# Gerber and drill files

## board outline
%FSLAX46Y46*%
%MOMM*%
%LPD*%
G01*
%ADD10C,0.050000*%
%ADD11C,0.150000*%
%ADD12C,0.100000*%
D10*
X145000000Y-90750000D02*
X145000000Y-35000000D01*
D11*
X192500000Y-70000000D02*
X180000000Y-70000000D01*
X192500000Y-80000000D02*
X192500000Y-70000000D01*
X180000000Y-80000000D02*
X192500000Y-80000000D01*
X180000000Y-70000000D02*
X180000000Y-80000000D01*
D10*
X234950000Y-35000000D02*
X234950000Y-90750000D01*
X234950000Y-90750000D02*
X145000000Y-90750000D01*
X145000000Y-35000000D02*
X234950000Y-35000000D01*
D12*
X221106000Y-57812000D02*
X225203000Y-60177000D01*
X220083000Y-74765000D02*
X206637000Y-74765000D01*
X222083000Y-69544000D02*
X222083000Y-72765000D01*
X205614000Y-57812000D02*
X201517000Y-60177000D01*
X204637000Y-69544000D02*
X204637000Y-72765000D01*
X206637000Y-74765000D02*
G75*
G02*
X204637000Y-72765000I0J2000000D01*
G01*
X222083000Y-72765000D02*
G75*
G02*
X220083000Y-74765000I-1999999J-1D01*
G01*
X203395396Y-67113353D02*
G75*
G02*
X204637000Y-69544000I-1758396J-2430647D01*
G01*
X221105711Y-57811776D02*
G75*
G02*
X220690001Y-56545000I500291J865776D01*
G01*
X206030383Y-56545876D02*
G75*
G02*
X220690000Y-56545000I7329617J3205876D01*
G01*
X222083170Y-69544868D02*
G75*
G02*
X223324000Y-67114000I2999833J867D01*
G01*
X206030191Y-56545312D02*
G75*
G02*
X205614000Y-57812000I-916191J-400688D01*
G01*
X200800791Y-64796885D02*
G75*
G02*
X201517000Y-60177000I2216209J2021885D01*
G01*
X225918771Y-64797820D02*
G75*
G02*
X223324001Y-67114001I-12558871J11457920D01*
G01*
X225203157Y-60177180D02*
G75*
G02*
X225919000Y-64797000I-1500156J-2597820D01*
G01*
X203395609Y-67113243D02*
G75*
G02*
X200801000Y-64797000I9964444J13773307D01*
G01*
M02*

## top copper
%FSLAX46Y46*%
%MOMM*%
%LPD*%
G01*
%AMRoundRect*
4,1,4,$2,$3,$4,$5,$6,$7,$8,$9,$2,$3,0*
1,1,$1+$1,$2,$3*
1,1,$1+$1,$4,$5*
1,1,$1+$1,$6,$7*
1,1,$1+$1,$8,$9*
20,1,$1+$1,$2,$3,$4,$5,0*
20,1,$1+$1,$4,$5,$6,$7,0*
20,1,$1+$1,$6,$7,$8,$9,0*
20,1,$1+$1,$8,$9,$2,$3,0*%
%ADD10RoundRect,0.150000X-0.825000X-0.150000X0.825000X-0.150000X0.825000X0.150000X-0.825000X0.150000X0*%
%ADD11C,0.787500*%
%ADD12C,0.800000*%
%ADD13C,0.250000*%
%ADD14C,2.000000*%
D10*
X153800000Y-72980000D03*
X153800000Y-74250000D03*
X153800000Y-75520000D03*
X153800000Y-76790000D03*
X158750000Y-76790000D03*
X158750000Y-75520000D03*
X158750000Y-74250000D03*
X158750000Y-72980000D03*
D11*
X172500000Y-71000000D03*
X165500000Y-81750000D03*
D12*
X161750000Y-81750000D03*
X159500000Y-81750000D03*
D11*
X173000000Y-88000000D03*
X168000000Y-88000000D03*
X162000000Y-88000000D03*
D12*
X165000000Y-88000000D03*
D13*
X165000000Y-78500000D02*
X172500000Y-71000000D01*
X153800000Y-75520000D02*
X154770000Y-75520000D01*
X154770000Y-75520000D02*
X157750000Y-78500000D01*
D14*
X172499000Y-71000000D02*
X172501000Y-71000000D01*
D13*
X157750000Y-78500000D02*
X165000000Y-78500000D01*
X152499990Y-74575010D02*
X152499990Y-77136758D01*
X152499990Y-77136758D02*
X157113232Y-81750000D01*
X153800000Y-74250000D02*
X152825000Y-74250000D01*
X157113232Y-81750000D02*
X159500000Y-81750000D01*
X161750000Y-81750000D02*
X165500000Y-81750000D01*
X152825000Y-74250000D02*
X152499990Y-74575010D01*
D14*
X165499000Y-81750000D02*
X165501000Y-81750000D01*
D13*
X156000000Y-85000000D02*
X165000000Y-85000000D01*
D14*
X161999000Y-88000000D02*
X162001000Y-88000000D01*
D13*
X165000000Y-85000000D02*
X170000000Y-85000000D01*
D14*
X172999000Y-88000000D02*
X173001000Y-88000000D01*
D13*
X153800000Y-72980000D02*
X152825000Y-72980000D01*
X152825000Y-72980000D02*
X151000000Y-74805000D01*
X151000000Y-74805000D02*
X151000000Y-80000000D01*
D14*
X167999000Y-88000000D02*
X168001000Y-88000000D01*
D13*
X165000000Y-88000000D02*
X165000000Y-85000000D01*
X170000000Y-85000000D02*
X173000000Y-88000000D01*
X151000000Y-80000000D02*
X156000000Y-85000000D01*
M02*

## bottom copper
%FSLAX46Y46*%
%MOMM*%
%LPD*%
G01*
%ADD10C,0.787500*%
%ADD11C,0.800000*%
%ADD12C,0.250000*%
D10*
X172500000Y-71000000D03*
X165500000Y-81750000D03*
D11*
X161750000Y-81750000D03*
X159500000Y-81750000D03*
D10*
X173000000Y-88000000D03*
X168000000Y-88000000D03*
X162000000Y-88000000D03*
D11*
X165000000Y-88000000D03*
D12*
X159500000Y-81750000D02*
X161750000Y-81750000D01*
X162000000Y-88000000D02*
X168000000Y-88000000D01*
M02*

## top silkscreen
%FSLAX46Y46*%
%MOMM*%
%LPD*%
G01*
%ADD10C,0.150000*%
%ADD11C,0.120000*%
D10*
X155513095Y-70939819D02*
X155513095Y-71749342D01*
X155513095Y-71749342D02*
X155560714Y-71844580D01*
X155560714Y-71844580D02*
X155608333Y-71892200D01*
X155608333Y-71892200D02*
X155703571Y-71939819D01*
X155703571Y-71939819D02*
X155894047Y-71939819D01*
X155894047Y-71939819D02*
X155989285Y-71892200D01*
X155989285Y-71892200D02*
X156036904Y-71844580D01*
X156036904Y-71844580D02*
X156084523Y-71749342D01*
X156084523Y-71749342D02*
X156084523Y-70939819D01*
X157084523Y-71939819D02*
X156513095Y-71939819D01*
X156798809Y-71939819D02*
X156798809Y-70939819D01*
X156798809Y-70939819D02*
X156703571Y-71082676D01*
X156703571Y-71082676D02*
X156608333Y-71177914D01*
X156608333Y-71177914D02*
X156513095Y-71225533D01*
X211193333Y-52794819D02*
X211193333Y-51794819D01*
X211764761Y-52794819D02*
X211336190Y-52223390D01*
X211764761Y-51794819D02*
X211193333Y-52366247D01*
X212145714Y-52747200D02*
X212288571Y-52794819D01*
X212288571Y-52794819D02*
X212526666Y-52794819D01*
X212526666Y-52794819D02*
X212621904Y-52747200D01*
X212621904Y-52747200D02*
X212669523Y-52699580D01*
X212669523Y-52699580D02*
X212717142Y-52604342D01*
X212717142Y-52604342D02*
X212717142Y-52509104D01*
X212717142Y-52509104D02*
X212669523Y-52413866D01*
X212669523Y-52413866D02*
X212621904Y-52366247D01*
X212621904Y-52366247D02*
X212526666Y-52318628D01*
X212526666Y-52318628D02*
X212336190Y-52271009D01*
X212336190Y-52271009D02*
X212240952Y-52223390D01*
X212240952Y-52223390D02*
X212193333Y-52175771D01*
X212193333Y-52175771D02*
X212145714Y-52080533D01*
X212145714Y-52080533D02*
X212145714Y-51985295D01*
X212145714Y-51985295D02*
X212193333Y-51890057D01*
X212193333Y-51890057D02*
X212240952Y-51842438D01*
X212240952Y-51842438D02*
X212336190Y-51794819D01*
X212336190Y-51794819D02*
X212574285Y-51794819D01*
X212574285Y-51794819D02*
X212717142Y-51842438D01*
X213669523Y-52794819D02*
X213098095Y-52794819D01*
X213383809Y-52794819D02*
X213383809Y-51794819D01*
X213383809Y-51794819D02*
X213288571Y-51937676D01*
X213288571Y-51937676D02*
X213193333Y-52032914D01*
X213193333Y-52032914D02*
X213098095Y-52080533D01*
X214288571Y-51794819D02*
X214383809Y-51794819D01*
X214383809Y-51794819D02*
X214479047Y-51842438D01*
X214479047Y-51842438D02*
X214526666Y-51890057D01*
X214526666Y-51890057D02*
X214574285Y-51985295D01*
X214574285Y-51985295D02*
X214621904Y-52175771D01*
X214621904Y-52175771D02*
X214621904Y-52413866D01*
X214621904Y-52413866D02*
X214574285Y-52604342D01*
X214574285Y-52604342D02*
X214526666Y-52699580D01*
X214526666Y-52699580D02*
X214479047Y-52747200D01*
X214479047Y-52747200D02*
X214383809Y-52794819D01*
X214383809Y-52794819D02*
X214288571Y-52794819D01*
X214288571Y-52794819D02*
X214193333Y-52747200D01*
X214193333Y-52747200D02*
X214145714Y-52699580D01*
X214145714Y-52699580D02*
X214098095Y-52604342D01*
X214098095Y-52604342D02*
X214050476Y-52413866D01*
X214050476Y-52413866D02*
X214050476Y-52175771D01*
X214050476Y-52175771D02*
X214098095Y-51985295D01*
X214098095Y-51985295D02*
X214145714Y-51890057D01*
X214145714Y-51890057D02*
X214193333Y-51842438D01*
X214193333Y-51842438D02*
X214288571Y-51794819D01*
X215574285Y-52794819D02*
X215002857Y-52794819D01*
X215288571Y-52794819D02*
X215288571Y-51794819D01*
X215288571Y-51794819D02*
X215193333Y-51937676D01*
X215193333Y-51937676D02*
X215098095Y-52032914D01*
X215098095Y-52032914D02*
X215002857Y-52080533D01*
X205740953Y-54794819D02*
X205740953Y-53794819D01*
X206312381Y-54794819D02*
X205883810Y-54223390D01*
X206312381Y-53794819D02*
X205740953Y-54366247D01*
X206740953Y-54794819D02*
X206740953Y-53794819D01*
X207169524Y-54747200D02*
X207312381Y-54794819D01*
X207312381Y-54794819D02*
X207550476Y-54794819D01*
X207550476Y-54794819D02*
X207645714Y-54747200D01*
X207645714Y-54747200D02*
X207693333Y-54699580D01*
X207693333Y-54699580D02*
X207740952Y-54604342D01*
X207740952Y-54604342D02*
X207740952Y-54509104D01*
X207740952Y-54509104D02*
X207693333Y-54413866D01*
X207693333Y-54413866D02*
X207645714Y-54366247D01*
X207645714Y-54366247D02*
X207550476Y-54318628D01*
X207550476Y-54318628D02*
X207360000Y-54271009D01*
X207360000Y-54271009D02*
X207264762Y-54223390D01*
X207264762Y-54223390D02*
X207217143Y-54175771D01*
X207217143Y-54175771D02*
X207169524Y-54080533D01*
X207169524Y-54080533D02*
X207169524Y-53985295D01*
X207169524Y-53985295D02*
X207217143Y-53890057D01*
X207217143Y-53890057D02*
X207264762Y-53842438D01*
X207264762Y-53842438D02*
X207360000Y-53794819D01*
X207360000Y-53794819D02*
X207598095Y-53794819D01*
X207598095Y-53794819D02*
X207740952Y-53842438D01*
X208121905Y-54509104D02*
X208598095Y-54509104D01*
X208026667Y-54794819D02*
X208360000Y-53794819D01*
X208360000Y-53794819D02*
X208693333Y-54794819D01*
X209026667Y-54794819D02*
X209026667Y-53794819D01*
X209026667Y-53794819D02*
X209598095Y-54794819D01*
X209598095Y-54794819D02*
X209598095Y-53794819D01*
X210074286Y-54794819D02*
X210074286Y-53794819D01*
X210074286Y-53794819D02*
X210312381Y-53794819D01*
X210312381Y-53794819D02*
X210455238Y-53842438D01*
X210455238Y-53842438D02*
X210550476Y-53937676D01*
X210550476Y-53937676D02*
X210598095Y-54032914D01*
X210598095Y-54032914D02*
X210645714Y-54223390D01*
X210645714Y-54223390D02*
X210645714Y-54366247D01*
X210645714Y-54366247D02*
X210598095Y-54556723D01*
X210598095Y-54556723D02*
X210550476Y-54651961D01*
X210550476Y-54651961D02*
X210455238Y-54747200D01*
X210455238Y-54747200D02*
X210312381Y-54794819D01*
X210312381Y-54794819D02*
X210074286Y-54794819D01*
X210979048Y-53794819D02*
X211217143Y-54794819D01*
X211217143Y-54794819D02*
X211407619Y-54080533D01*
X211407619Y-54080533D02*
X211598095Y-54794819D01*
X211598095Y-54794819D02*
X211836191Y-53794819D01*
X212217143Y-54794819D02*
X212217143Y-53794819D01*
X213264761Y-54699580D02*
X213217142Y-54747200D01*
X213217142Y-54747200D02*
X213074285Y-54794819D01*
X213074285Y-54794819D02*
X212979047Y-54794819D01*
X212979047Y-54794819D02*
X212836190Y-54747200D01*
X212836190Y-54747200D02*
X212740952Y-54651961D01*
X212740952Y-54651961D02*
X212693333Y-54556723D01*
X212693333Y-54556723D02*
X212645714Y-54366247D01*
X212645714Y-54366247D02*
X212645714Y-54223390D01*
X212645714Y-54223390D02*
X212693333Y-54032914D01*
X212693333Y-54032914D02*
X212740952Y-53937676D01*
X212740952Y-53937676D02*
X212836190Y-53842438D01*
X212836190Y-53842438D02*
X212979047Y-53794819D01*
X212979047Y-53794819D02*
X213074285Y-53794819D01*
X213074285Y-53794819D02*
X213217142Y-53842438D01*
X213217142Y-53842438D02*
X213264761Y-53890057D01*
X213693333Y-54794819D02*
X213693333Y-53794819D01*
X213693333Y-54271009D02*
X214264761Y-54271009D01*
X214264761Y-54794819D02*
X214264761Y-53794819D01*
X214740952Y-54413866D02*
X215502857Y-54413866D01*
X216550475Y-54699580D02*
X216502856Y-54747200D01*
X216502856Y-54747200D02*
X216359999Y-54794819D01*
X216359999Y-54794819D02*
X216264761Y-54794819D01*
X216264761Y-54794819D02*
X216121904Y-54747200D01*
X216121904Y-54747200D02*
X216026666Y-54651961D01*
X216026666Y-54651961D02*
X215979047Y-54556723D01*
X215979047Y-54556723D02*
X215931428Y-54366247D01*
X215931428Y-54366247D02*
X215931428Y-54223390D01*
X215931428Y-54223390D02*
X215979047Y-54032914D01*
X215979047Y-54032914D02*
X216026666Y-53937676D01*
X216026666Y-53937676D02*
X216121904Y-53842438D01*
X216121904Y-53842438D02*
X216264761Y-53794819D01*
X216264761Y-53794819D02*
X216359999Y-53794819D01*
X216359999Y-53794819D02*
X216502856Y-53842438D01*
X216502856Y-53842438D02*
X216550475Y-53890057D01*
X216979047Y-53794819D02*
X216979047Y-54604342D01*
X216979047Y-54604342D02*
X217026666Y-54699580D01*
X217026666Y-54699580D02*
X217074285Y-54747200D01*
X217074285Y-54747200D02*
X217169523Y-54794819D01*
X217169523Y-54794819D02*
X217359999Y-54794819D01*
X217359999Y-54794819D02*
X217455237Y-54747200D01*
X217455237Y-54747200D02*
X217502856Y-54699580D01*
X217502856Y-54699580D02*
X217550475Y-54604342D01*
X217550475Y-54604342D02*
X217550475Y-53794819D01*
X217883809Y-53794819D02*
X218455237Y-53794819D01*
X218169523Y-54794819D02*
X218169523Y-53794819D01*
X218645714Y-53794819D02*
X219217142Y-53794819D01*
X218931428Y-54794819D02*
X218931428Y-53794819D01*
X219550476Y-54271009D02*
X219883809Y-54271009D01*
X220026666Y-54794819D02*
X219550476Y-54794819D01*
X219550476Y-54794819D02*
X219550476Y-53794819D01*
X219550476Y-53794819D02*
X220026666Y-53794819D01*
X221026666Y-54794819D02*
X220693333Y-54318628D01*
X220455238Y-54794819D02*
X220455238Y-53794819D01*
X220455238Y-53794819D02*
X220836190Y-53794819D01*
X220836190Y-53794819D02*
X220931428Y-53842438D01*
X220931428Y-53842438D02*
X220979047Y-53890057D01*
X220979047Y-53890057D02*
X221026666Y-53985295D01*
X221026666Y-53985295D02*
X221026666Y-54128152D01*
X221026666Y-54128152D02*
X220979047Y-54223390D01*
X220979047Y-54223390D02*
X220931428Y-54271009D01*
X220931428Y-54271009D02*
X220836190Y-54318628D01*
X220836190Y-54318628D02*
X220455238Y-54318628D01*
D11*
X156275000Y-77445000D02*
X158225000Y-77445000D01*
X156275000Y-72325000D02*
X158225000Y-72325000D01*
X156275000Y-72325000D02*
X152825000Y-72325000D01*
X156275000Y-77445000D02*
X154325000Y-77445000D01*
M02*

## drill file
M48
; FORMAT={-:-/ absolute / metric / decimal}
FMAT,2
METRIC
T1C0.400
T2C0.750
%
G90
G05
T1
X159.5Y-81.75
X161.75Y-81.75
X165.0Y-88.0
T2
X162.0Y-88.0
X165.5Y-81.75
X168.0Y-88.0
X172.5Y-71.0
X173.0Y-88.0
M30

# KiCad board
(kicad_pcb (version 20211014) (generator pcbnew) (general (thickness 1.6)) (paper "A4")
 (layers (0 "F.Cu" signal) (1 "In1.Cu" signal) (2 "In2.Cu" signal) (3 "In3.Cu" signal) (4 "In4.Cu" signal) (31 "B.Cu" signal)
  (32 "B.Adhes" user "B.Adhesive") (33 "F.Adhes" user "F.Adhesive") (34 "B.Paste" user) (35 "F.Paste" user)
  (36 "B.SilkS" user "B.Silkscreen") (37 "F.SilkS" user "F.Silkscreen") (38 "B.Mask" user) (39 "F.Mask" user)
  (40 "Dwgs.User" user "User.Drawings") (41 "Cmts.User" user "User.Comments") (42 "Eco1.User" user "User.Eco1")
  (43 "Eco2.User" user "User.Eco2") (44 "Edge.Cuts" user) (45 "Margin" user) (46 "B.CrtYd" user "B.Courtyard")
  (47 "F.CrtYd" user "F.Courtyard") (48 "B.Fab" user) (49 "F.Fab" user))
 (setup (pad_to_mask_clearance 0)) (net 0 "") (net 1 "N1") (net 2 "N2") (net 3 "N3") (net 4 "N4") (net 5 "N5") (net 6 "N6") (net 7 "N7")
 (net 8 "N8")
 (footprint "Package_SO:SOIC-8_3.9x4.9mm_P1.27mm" (layer "F.Cu") (at 156.275 74.885)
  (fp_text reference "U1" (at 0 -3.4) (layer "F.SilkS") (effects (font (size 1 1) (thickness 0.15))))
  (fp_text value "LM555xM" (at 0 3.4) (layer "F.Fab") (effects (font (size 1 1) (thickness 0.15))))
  (fp_line (start 0 2.56) (end 1.95 2.56) (layer "F.SilkS") (width 0.12))
  (fp_line (start 0 -2.56) (end 1.95 -2.56) (layer "F.SilkS") (width 0.12))
  (fp_line (start 0 -2.56) (end -3.45 -2.56) (layer "F.SilkS") (width 0.12))
  (fp_line (start 0 2.56) (end -1.95 2.56) (layer "F.SilkS") (width 0.12))
  (pad "1" smd roundrect locked (at -2.475 -1.905) (size 1.95 0.6) (layers "F.Cu" "F.Paste" "F.Mask") (roundrect_rratio 0.25) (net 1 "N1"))
  (pad "2" smd roundrect locked (at -2.475 -0.635) (size 1.95 0.6) (layers "F.Cu" "F.Paste" "F.Mask") (roundrect_rratio 0.25) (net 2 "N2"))
  (pad "3" smd roundrect locked (at -2.475 0.635) (size 1.95 0.6) (layers "F.Cu" "F.Paste" "F.Mask") (roundrect_rratio 0.25) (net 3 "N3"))
  (pad "4" smd roundrect locked (at -2.475 1.905) (size 1.95 0.6) (layers "F.Cu" "F.Paste" "F.Mask") (roundrect_rratio 0.25) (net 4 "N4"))
  (pad "5" smd roundrect locked (at 2.475 1.905) (size 1.95 0.6) (layers "F.Cu" "F.Paste" "F.Mask") (roundrect_rratio 0.25) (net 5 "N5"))
  (pad "6" smd roundrect locked (at 2.475 0.635) (size 1.95 0.6) (layers "F.Cu" "F.Paste" "F.Mask") (roundrect_rratio 0.25) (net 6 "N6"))
  (pad "7" smd roundrect locked (at 2.475 -0.635) (size 1.95 0.6) (layers "F.Cu" "F.Paste" "F.Mask") (roundrect_rratio 0.25) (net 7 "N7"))
  (pad "8" smd roundrect locked (at 2.475 -1.905) (size 1.95 0.6) (layers "F.Cu" "F.Paste" "F.Mask") (roundrect_rratio 0.25) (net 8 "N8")))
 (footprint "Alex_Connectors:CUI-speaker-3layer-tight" (layer "F.Cu") (at 213.36 53.34 180)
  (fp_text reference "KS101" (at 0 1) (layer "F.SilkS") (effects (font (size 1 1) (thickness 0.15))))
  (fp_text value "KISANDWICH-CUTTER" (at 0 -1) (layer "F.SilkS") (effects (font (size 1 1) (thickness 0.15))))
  (fp_line (start -7.746 -4.472) (end -11.843 -6.837) (layer "Edge.Cuts") (width 0.1))
  (fp_line (start -6.723 -21.425) (end 6.723 -21.425) (layer "Edge.Cuts") (width 0.1))
  (fp_line (start -8.723 -16.204) (end -8.723 -19.425) (layer "Edge.Cuts") (width 0.1))
  (fp_line (start 7.746 -4.472) (end 11.843 -6.837) (layer "Edge.Cuts") (width 0.1))
  (fp_line (start 8.723 -16.204) (end 8.723 -19.425) (layer "Edge.Cuts") (width 0.1))
  (fp_arc (start 6.723 -21.425) (mid 8.137214 -20.839214) (end 8.723 -19.425) (layer "Edge.Cuts") (width 0.1))
  (fp_arc (start -8.723 -19.425) (mid -8.137214 -20.839214) (end -6.723 -21.425) (layer "Edge.Cuts") (width 0.1))
  (fp_arc (start 9.964604 -13.773353) (mid 9.051372 -14.8393) (end 8.723 -16.204) (layer "Edge.Cuts") (width 0.1))
  (fp_arc (start -7.745711 -4.471776) (mid -7.295922 -3.917782) (end -7.33 -3.205) (layer "Edge.Cuts") (width 0.1))
  (fp_arc (start 7.329617 -3.205876) (mid 0.000478 8.000058) (end -7.33 -3.205) (layer "Edge.Cuts") (width 0.1))
  (fp_arc (start -8.72317 -16.204868) (mid -9.051129 -14.840151) (end -9.964 -13.774) (layer "Edge.Cuts") (width 0.1))
  (fp_arc (start 7.329809 -3.205312) (mid 7.295987 -3.918142) (end 7.746 -4.472) (layer "Edge.Cuts") (width 0.1))
  (fp_arc (start 12.559209 -11.456885) (mid 13.307521 -8.975418) (end 11.843 -6.837) (layer "Edge.Cuts") (width 0.1))
  (fp_arc (start -12.558771 -11.45782) (mid -11.320776 -12.682444) (end -9.964 -13.774) (layer "Edge.Cuts") (width 0.1))
  (fp_arc (start -11.843157 -6.83718) (mid -13.30748 -8.975653) (end -12.559 -11.457) (layer "Edge.Cuts") (width 0.1))
  (fp_arc (start 9.964391 -13.773243) (mid 11.321088 -12.681651) (end 12.559 -11.457) (layer "Edge.Cuts") (width 0.1)))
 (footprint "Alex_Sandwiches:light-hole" (layer "F.Cu") (at 201.93 77.47)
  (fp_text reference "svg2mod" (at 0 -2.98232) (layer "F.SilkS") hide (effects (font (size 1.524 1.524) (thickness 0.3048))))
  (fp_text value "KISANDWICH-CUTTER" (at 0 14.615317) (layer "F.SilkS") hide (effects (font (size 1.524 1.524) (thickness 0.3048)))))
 (gr_line (start 145 90.75) (end 145 35) (layer "Edge.Cuts") (width 0.05))
 (gr_line (start 192.5 70) (end 180 70) (layer "Edge.Cuts") (width 0.15))
 (gr_line (start 192.5 80) (end 192.5 70) (layer "Edge.Cuts") (width 0.15))
 (gr_line (start 180 80) (end 192.5 80) (layer "Edge.Cuts") (width 0.15))
 (gr_line (start 180 70) (end 180 80) (layer "Edge.Cuts") (width 0.15))
 (gr_line (start 234.95 35) (end 234.95 90.75) (layer "Edge.Cuts") (width 0.05))
 (gr_line (start 234.95 90.75) (end 145 90.75) (layer "Edge.Cuts") (width 0.05))
 (gr_line (start 145 35) (end 234.95 35) (layer "Edge.Cuts") (width 0.05))
 (segment (start 165 78.5) (end 172.5 71) (width 0.25) (layer "F.Cu") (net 3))
 (segment (start 153.8 75.52) (end 154.77 75.52) (width 0.25) (layer "F.Cu") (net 3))
 (segment (start 154.77 75.52) (end 157.75 78.5) (width 0.25) (layer "F.Cu") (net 3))
 (segment (start 172.499 71) (end 172.501 71) (width 2) (layer "F.Cu") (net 3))
 (segment (start 157.75 78.5) (end 165 78.5) (width 0.25) (layer "F.Cu") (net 3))
 (via (at 172.5 71) (size 0.7875) (drill 0.75) (layers "F.Cu" "B.Cu") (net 3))
 (segment (start 152.49999 74.57501) (end 152.49999 77.136758) (width 0.25) (layer "F.Cu") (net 2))
 (segment (start 152.49999 77.136758) (end 157.113232 81.75) (width 0.25) (layer "F.Cu") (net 2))
 (segment (start 153.8 74.25) (end 152.825 74.25) (width 0.25) (layer "F.Cu") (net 2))
 (segment (start 157.113232 81.75) (end 159.5 81.75) (width 0.25) (layer "F.Cu") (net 2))
 (segment (start 161.75 81.75) (end 165.5 81.75) (width 0.25) (layer "F.Cu") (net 2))
 (segment (start 152.825 74.25) (end 152.49999 74.57501) (width 0.25) (layer "F.Cu") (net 2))
 (segment (start 165.499 81.75) (end 165.501 81.75) (width 2) (layer "F.Cu") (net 2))
 (via (at 165.5 81.75) (size 0.7875) (drill 0.75) (layers "F.Cu" "B.Cu") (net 2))
 (segment (start 159.5 81.75) (end 161.75 81.75) (width 0.25) (layer "B.Cu") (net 2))
 (via (at 161.75 81.75) (size 0.8) (drill 0.4) (layers "F.Cu" "B.Cu") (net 2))
 (via (at 159.5 81.75) (size 0.8) (drill 0.4) (layers "F.Cu" "B.Cu") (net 2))
 (segment (start 156 85) (end 165 85) (width 0.25) (layer "F.Cu") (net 1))
 (segment (start 161.999 88) (end 162.001 88) (width 2) (layer "F.Cu") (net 1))
 (segment (start 165 85) (end 170 85) (width 0.25) (layer "F.Cu") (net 1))
 (segment (start 172.999 88) (end 173.001 88) (width 2) (layer "F.Cu") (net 1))
 (segment (start 153.8 72.98) (end 152.825 72.98) (width 0.25) (layer "F.Cu") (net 1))
 (segment (start 152.825 72.98) (end 151 74.805) (width 0.25) (layer "F.Cu") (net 1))
 (segment (start 151 74.805) (end 151 80) (width 0.25) (layer "F.Cu") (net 1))
 (segment (start 167.999 88) (end 168.001 88) (width 2) (layer "F.Cu") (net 1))
 (segment (start 165 88) (end 165 85) (width 0.25) (layer "F.Cu") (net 1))
 (segment (start 170 85) (end 173 88) (width 0.25) (layer "F.Cu") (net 1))
 (segment (start 151 80) (end 156 85) (width 0.25) (layer "F.Cu") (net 1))
 (via (at 173 88) (size 0.7875) (drill 0.75) (layers "F.Cu" "B.Cu") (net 1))
 (via (at 168 88) (size 0.7875) (drill 0.75) (layers "F.Cu" "B.Cu") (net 1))
 (via (at 162 88) (size 0.7875) (drill 0.75) (layers "F.Cu" "B.Cu") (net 1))
 (segment (start 162 88) (end 168 88) (width 0.25) (layer "B.Cu") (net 1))
 (via (at 165 88) (size 0.8) (drill 0.4) (layers "F.Cu" "B.Cu") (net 1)))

